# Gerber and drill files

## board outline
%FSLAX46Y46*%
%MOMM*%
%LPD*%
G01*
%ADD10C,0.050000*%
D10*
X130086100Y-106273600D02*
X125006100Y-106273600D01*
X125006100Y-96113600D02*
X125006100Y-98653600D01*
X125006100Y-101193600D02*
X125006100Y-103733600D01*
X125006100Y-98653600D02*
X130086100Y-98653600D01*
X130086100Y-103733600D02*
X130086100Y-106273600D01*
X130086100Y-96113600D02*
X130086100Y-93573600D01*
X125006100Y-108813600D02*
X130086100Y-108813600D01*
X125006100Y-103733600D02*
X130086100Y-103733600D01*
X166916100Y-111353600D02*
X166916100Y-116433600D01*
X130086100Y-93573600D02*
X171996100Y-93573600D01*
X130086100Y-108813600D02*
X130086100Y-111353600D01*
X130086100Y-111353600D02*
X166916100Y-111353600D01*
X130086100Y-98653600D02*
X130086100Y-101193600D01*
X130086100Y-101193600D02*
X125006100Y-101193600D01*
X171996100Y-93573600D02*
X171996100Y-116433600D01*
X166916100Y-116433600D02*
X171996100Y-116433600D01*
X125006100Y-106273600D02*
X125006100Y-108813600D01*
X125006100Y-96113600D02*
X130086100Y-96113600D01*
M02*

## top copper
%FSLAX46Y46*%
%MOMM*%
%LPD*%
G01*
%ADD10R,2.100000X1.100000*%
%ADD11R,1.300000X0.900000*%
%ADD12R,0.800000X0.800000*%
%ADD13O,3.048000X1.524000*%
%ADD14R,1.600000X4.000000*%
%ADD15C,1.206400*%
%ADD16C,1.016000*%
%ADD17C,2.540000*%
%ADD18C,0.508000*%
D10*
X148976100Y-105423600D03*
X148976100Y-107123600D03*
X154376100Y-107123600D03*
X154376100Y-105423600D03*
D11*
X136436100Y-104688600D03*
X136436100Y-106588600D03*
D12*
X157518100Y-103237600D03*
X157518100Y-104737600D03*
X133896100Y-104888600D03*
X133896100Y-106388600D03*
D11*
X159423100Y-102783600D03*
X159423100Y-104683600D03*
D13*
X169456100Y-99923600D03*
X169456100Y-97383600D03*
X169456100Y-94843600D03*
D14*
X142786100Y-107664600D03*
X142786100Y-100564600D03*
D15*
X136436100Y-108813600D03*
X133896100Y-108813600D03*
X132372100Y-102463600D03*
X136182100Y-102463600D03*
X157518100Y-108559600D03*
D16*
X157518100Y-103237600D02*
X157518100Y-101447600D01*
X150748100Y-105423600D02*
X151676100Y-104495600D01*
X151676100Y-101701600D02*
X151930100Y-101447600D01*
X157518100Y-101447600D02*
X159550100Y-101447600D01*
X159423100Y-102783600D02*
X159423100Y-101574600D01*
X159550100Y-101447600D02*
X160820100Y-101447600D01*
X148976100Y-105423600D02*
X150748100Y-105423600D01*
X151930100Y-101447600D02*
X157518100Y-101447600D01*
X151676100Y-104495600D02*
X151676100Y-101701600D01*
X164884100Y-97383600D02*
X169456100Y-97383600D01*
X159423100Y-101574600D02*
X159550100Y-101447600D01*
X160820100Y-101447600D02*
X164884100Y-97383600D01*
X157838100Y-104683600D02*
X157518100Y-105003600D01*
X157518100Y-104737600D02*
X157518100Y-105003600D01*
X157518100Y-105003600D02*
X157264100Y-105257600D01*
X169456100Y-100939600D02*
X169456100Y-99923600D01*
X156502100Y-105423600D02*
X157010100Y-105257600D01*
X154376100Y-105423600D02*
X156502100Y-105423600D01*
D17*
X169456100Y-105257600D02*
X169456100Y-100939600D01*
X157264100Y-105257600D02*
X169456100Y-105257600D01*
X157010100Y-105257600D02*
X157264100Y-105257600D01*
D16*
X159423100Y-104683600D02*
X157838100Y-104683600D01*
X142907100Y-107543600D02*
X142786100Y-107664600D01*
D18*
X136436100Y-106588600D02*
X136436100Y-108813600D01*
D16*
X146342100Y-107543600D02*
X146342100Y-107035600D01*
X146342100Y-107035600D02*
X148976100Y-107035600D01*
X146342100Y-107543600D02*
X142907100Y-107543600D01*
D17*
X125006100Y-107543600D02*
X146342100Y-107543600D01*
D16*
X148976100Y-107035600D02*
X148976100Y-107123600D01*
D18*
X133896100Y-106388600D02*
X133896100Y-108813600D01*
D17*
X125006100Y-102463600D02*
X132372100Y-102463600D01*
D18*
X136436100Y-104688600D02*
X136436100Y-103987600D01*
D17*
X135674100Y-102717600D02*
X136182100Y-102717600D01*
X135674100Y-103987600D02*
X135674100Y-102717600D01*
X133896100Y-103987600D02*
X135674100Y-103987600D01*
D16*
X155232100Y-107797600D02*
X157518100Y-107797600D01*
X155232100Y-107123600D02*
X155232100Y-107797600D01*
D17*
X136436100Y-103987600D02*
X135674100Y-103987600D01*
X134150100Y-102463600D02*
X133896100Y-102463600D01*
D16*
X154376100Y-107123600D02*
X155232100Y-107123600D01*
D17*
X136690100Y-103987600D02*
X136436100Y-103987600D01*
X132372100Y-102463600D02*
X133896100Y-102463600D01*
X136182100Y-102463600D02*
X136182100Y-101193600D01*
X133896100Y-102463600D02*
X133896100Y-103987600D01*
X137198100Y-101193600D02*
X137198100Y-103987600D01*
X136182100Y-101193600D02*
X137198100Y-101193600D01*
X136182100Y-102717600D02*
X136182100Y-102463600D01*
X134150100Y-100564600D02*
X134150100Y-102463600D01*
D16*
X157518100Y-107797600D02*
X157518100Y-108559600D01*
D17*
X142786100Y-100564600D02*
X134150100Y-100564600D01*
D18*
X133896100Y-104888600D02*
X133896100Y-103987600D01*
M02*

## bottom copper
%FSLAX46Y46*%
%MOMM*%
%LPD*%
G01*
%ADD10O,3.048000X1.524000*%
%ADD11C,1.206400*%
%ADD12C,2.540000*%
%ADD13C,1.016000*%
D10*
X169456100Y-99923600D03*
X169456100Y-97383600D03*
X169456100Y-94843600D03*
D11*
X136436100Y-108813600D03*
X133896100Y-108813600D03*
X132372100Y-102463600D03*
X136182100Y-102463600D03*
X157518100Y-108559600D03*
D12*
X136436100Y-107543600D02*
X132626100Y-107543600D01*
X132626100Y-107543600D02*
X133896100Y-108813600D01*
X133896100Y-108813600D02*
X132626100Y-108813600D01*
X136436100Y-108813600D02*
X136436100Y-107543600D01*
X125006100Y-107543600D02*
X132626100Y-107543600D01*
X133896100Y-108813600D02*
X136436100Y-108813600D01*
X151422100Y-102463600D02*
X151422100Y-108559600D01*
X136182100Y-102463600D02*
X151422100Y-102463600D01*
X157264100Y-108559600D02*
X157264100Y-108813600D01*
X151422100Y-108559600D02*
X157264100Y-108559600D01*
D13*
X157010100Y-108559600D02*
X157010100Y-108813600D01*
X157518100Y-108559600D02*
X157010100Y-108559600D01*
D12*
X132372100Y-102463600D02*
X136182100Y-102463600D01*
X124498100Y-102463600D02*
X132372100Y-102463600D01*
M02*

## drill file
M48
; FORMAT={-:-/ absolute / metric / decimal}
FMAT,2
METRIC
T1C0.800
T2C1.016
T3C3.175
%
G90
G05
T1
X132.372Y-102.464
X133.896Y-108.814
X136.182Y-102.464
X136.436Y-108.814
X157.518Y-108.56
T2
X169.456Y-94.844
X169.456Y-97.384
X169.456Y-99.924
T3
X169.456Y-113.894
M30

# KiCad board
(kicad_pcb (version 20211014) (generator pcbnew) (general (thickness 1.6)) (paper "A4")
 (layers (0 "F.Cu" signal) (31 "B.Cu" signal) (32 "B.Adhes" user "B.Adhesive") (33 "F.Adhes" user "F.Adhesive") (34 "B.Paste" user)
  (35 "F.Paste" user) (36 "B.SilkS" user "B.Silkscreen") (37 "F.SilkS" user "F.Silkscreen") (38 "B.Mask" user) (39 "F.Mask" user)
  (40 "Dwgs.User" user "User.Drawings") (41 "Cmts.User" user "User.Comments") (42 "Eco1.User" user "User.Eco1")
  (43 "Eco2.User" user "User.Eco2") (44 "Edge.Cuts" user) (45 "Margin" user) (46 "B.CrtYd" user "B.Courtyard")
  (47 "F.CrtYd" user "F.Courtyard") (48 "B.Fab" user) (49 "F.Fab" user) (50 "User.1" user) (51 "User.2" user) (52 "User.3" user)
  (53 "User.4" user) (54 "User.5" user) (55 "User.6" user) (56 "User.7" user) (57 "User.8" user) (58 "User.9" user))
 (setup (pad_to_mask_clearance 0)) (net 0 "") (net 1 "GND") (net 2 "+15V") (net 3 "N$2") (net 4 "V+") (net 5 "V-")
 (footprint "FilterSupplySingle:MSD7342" (layer "F.Cu") (at 151.6761 106.2736)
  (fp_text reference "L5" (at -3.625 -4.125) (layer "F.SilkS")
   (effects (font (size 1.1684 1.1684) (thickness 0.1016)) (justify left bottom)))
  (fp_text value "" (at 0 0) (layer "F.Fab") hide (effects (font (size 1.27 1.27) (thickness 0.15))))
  (pad "1" smd rect (at -2.7 -0.85) (size 2.1 1.1) (layers "F.Cu" "F.Paste" "F.Mask") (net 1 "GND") (solder_mask_margin 0.1016))
  (pad "2" smd rect (at -2.7 0.85) (size 2.1 1.1) (layers "F.Cu" "F.Paste" "F.Mask") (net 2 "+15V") (solder_mask_margin 0.1016))
  (pad "3" smd rect (at 2.7 0.85) (size 2.1 1.1) (layers "F.Cu" "F.Paste" "F.Mask") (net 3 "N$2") (solder_mask_margin 0.1016))
  (pad "4" smd rect (at 2.7 -0.85) (size 2.1 1.1) (layers "F.Cu" "F.Paste" "F.Mask") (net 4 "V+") (solder_mask_margin 0.1016)))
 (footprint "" (layer "F.Cu") (at 169.4561 113.8936)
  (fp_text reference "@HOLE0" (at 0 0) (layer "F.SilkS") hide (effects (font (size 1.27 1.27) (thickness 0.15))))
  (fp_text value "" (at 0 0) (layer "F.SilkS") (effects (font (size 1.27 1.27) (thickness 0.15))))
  (pad "" np_thru_hole circle (at 0 0) (size 3.175 3.175) (drill 3.175) (layers *.Cu *.Mask)))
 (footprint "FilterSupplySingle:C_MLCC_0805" (layer "F.Cu") (at 136.4361 105.6386 -90)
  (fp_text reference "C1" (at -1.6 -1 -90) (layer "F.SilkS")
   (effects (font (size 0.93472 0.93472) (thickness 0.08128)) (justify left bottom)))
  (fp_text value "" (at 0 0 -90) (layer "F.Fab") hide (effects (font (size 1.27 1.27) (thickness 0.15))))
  (pad "P$1" smd rect (at -0.95 0 270) (size 0.9 1.3) (layers "F.Cu" "F.Paste" "F.Mask") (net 3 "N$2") (solder_mask_margin 0.1016))
  (pad "P$2" smd rect (at 0.95 0 270) (size 0.9 1.3) (layers "F.Cu" "F.Paste" "F.Mask") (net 2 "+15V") (solder_mask_margin 0.1016)))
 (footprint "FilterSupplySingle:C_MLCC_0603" (layer "F.Cu") (at 157.5181 103.9876 -90)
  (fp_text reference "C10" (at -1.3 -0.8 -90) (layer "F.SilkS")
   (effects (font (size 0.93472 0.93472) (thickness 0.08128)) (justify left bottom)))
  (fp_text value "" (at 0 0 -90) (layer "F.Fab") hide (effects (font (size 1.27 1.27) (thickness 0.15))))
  (pad "P$1" smd rect (at -0.75 0 270) (size 0.8 0.8) (layers "F.Cu" "F.Paste" "F.Mask") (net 1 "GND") (solder_mask_margin 0.1016))
  (pad "P$2" smd rect (at 0.75 0 270) (size 0.8 0.8) (layers "F.Cu" "F.Paste" "F.Mask") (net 4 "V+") (solder_mask_margin 0.1016)))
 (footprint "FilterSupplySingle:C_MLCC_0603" (layer "F.Cu") (at 133.8961 105.6386 -90)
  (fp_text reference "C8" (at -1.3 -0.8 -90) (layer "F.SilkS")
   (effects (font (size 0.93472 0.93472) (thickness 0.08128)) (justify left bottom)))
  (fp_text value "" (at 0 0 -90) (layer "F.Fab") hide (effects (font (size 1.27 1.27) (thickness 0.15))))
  (pad "P$1" smd rect (at -0.75 0 270) (size 0.8 0.8) (layers "F.Cu" "F.Paste" "F.Mask") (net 3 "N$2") (solder_mask_margin 0.1016))
  (pad "P$2" smd rect (at 0.75 0 270) (size 0.8 0.8) (layers "F.Cu" "F.Paste" "F.Mask") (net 2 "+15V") (solder_mask_margin 0.1016)))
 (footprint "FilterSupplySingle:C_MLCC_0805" (layer "F.Cu") (at 159.4231 103.7336 -90)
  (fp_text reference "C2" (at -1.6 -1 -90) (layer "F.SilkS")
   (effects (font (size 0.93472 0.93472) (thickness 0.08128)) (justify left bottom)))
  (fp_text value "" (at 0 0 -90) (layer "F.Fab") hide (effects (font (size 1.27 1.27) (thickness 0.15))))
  (pad "P$1" smd rect (at -0.95 0 270) (size 0.9 1.3) (layers "F.Cu" "F.Paste" "F.Mask") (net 1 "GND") (solder_mask_margin 0.1016))
  (pad "P$2" smd rect (at 0.95 0 270) (size 0.9 1.3) (layers "F.Cu" "F.Paste" "F.Mask") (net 4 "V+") (solder_mask_margin 0.1016)))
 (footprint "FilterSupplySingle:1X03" (layer "F.Cu") (at 169.4561 97.3836 90)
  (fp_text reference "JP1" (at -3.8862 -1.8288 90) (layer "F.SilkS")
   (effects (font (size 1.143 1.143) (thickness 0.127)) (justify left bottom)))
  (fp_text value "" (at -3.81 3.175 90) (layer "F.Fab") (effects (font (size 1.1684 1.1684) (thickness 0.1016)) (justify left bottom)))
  (pad "1" thru_hole oval (at -2.54 0 180) (size 3.048 1.524) (drill 1.016) (layers *.Cu *.Mask) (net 4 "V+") (solder_mask_margin 0.1016))
  (pad "2" thru_hole oval (at 0 0 180) (size 3.048 1.524) (drill 1.016) (layers *.Cu *.Mask) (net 1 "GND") (solder_mask_margin 0.1016))
  (pad "3" thru_hole oval (at 2.54 0 180) (size 3.048 1.524) (drill 1.016) (layers *.Cu *.Mask) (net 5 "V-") (solder_mask_margin 0.1016)))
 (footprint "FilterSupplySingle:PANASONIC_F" (layer "F.Cu") (at 142.7861 104.1146 -90)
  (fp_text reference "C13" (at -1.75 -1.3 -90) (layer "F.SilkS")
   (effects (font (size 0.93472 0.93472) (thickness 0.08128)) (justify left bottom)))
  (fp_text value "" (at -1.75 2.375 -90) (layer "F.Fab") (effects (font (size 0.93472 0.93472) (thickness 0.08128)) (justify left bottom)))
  (pad "+" smd rect (at 3.55 0 270) (size 4 1.6) (layers "F.Cu" "F.Paste" "F.Mask") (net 2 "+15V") (solder_mask_margin 0.1016))
  (pad "-" smd rect (at -3.55 0 270) (size 4 1.6) (layers "F.Cu" "F.Paste" "F.Mask") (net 3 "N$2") (solder_mask_margin 0.1016)))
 (gr_line (start 130.0861 106.2736) (end 125.0061 106.2736) (layer "Edge.Cuts") (width 0.05))
 (gr_line (start 125.0061 96.1136) (end 125.0061 98.6536) (layer "Edge.Cuts") (width 0.05))
 (gr_line (start 125.0061 101.1936) (end 125.0061 103.7336) (layer "Edge.Cuts") (width 0.05))
 (gr_line (start 125.0061 98.6536) (end 130.0861 98.6536) (layer "Edge.Cuts") (width 0.05))
 (gr_line (start 130.0861 103.7336) (end 130.0861 106.2736) (layer "Edge.Cuts") (width 0.05))
 (gr_line (start 130.0861 96.1136) (end 130.0861 93.5736) (layer "Edge.Cuts") (width 0.05))
 (gr_line (start 125.0061 108.8136) (end 130.0861 108.8136) (layer "Edge.Cuts") (width 0.05))
 (gr_line (start 125.0061 103.7336) (end 130.0861 103.7336) (layer "Edge.Cuts") (width 0.05))
 (gr_line (start 166.9161 111.3536) (end 166.9161 116.4336) (layer "Edge.Cuts") (width 0.05))
 (gr_line (start 130.0861 93.5736) (end 171.9961 93.5736) (layer "Edge.Cuts") (width 0.05))
 (gr_line (start 130.0861 108.8136) (end 130.0861 111.3536) (layer "Edge.Cuts") (width 0.05))
 (gr_line (start 130.0861 111.3536) (end 166.9161 111.3536) (layer "Edge.Cuts") (width 0.05))
 (gr_line (start 130.0861 98.6536) (end 130.0861 101.1936) (layer "Edge.Cuts") (width 0.05))
 (gr_line (start 130.0861 101.1936) (end 125.0061 101.1936) (layer "Edge.Cuts") (width 0.05))
 (gr_line (start 171.9961 93.5736) (end 171.9961 116.4336) (layer "Edge.Cuts") (width 0.05))
 (gr_line (start 166.9161 116.4336) (end 171.9961 116.4336) (layer "Edge.Cuts") (width 0.05))
 (gr_line (start 125.0061 106.2736) (end 125.0061 108.8136) (layer "Edge.Cuts") (width 0.05))
 (gr_line (start 125.0061 96.1136) (end 130.0861 96.1136) (layer "Edge.Cuts") (width 0.05))
 (segment (start 157.5181 103.2376) (end 157.5181 101.4476) (width 1.016) (layer "F.Cu") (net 1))
 (segment (start 150.7481 105.4236) (end 151.6761 104.4956) (width 1.016) (layer "F.Cu") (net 1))
 (segment (start 151.6761 101.7016) (end 151.9301 101.4476) (width 1.016) (layer "F.Cu") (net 1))
 (segment (start 157.5181 101.4476) (end 159.5501 101.4476) (width 1.016) (layer "F.Cu") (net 1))
 (segment (start 159.4231 102.7836) (end 159.4231 101.5746) (width 1.016) (layer "F.Cu") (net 1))
 (segment (start 159.5501 101.4476) (end 160.8201 101.4476) (width 1.016) (layer "F.Cu") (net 1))
 (segment (start 148.9761 105.4236) (end 150.7481 105.4236) (width 1.016) (layer "F.Cu") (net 1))
 (segment (start 151.9301 101.4476) (end 157.5181 101.4476) (width 1.016) (layer "F.Cu") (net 1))
 (segment (start 151.6761 104.4956) (end 151.6761 101.7016) (width 1.016) (layer "F.Cu") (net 1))
 (segment (start 164.8841 97.3836) (end 169.4561 97.3836) (width 1.016) (layer "F.Cu") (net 1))
 (segment (start 159.4231 101.5746) (end 159.5501 101.4476) (width 1.016) (layer "F.Cu") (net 1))
 (segment (start 160.8201 101.4476) (end 164.8841 97.3836) (width 1.016) (layer "F.Cu") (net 1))
 (segment (start 157.8381 104.6836) (end 157.5181 105.0036) (width 1.016) (layer "F.Cu") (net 4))
 (segment (start 157.5181 104.7376) (end 157.5181 105.0036) (width 1.016) (layer "F.Cu") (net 4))
 (segment (start 157.5181 105.0036) (end 157.2641 105.2576) (width 1.016) (layer "F.Cu") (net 4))
 (segment (start 169.4561 100.9396) (end 169.4561 99.9236) (width 1.016) (layer "F.Cu") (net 4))
 (segment (start 156.5021 105.4236) (end 157.0101 105.2576) (width 1.016) (layer "F.Cu") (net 4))
 (segment (start 154.3761 105.4236) (end 156.5021 105.4236) (width 1.016) (layer "F.Cu") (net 4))
 (segment (start 169.4561 105.2576) (end 169.4561 100.9396) (width 2.54) (layer "F.Cu") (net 4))
 (segment (start 157.2641 105.2576) (end 169.4561 105.2576) (width 2.54) (layer "F.Cu") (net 4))
 (segment (start 157.0101 105.2576) (end 157.2641 105.2576) (width 2.54) (layer "F.Cu") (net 4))
 (segment (start 159.4231 104.6836) (end 157.8381 104.6836) (width 1.016) (layer "F.Cu") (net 4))
 (segment (start 142.9071 107.5436) (end 142.7861 107.6646) (width 1.016) (layer "F.Cu") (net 2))
 (segment (start 136.4361 106.5886) (end 136.4361 108.8136) (width 0.508) (layer "F.Cu") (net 2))
 (segment (start 146.3421 107.5436) (end 146.3421 107.0356) (width 1.016) (layer "F.Cu") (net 2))
 (segment (start 146.3421 107.0356) (end 148.9761 107.0356) (width 1.016) (layer "F.Cu") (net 2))
 (segment (start 146.3421 107.5436) (end 142.9071 107.5436) (width 1.016) (layer "F.Cu") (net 2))
 (segment (start 125.0061 107.5436) (end 146.3421 107.5436) (width 2.54) (layer "F.Cu") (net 2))
 (segment (start 148.9761 107.0356) (end 148.9761 107.1236) (width 1.016) (layer "F.Cu") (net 2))
 (segment (start 133.8961 106.3886) (end 133.8961 108.8136) (width 0.508) (layer "F.Cu") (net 2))
 (via (at 136.4361 108.8136) (size 1.2064) (drill 0.8) (layers "F.Cu" "B.Cu") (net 2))
 (via (at 133.8961 108.8136) (size 1.2064) (drill 0.8) (layers "F.Cu" "B.Cu") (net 2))
 (segment (start 136.4361 107.5436) (end 132.6261 107.5436) (width 2.54) (layer "B.Cu") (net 2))
 (segment (start 132.6261 107.5436) (end 133.8961 108.8136) (width 2.54) (layer "B.Cu") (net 2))
 (segment (start 133.8961 108.8136) (end 132.6261 108.8136) (width 2.54) (layer "B.Cu") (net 2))
 (segment (start 136.4361 108.8136) (end 136.4361 107.5436) (width 2.54) (layer "B.Cu") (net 2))
 (segment (start 125.0061 107.5436) (end 132.6261 107.5436) (width 2.54) (layer "B.Cu") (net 2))
 (segment (start 133.8961 108.8136) (end 136.4361 108.8136) (width 2.54) (layer "B.Cu") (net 2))
 (segment (start 125.0061 102.4636) (end 132.3721 102.4636) (width 2.54) (layer "F.Cu") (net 3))
 (segment (start 136.4361 104.6886) (end 136.4361 103.9876) (width 0.508) (layer "F.Cu") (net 3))
 (segment (start 135.6741 102.7176) (end 136.1821 102.7176) (width 2.54) (layer "F.Cu") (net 3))
 (segment (start 135.6741 103.9876) (end 135.6741 102.7176) (width 2.54) (layer "F.Cu") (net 3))
 (segment (start 133.8961 103.9876) (end 135.6741 103.9876) (width 2.54) (layer "F.Cu") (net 3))
 (segment (start 155.2321 107.7976) (end 157.5181 107.7976) (width 1.016) (layer "F.Cu") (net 3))
 (segment (start 155.2321 107.1236) (end 155.2321 107.7976) (width 1.016) (layer "F.Cu") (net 3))
 (segment (start 136.4361 103.9876) (end 135.6741 103.9876) (width 2.54) (layer "F.Cu") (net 3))
 (segment (start 134.1501 102.4636) (end 133.8961 102.4636) (width 2.54) (layer "F.Cu") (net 3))
 (segment (start 154.3761 107.1236) (end 155.2321 107.1236) (width 1.016) (layer "F.Cu") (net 3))
 (segment (start 136.6901 103.9876) (end 136.4361 103.9876) (width 2.54) (layer "F.Cu") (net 3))
 (segment (start 132.3721 102.4636) (end 133.8961 102.4636) (width 2.54) (layer "F.Cu") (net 3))
 (segment (start 136.1821 102.4636) (end 136.1821 101.1936) (width 2.54) (layer "F.Cu") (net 3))
 (segment (start 133.8961 102.4636) (end 133.8961 103.9876) (width 2.54) (layer "F.Cu") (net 3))
 (segment (start 137.1981 101.1936) (end 137.1981 103.9876) (width 2.54) (layer "F.Cu") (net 3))
 (segment (start 136.1821 101.1936) (end 137.1981 101.1936) (width 2.54) (layer "F.Cu") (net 3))
 (segment (start 136.1821 102.7176) (end 136.1821 102.4636) (width 2.54) (layer "F.Cu") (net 3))
 (segment (start 134.1501 100.5646) (end 134.1501 102.4636) (width 2.54) (layer "F.Cu") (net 3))
 (segment (start 157.5181 107.7976) (end 157.5181 108.5596) (width 1.016) (layer "F.Cu") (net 3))
 (segment (start 142.7861 100.5646) (end 134.1501 100.5646) (width 2.54) (layer "F.Cu") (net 3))
 (segment (start 133.8961 104.8886) (end 133.8961 103.9876) (width 0.508) (layer "F.Cu") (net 3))
 (via (at 132.3721 102.4636) (size 1.2064) (drill 0.8) (layers "F.Cu" "B.Cu") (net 3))
 (via (at 136.1821 102.4636) (size 1.2064) (drill 0.8) (layers "F.Cu" "B.Cu") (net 3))
 (via (at 157.5181 108.5596) (size 1.2064) (drill 0.8) (layers "F.Cu" "B.Cu") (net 3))
 (segment (start 151.4221 102.4636) (end 151.4221 108.5596) (width 2.54) (layer "B.Cu") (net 3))
 (segment (start 136.1821 102.4636) (end 151.4221 102.4636) (width 2.54) (layer "B.Cu") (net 3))
 (segment (start 157.2641 108.5596) (end 157.2641 108.8136) (width 2.54) (layer "B.Cu") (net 3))
 (segment (start 151.4221 108.5596) (end 157.2641 108.5596) (width 2.54) (layer "B.Cu") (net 3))
 (segment (start 157.0101 108.5596) (end 157.0101 108.8136) (width 1.016) (layer "B.Cu") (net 3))
 (segment (start 157.5181 108.5596) (end 157.0101 108.5596) (width 1.016) (layer "B.Cu") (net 3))
 (segment (start 132.3721 102.4636) (end 136.1821 102.4636) (width 2.54) (layer "B.Cu") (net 3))
 (segment (start 124.4981 102.4636) (end 132.3721 102.4636) (width 2.54) (layer "B.Cu") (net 3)))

